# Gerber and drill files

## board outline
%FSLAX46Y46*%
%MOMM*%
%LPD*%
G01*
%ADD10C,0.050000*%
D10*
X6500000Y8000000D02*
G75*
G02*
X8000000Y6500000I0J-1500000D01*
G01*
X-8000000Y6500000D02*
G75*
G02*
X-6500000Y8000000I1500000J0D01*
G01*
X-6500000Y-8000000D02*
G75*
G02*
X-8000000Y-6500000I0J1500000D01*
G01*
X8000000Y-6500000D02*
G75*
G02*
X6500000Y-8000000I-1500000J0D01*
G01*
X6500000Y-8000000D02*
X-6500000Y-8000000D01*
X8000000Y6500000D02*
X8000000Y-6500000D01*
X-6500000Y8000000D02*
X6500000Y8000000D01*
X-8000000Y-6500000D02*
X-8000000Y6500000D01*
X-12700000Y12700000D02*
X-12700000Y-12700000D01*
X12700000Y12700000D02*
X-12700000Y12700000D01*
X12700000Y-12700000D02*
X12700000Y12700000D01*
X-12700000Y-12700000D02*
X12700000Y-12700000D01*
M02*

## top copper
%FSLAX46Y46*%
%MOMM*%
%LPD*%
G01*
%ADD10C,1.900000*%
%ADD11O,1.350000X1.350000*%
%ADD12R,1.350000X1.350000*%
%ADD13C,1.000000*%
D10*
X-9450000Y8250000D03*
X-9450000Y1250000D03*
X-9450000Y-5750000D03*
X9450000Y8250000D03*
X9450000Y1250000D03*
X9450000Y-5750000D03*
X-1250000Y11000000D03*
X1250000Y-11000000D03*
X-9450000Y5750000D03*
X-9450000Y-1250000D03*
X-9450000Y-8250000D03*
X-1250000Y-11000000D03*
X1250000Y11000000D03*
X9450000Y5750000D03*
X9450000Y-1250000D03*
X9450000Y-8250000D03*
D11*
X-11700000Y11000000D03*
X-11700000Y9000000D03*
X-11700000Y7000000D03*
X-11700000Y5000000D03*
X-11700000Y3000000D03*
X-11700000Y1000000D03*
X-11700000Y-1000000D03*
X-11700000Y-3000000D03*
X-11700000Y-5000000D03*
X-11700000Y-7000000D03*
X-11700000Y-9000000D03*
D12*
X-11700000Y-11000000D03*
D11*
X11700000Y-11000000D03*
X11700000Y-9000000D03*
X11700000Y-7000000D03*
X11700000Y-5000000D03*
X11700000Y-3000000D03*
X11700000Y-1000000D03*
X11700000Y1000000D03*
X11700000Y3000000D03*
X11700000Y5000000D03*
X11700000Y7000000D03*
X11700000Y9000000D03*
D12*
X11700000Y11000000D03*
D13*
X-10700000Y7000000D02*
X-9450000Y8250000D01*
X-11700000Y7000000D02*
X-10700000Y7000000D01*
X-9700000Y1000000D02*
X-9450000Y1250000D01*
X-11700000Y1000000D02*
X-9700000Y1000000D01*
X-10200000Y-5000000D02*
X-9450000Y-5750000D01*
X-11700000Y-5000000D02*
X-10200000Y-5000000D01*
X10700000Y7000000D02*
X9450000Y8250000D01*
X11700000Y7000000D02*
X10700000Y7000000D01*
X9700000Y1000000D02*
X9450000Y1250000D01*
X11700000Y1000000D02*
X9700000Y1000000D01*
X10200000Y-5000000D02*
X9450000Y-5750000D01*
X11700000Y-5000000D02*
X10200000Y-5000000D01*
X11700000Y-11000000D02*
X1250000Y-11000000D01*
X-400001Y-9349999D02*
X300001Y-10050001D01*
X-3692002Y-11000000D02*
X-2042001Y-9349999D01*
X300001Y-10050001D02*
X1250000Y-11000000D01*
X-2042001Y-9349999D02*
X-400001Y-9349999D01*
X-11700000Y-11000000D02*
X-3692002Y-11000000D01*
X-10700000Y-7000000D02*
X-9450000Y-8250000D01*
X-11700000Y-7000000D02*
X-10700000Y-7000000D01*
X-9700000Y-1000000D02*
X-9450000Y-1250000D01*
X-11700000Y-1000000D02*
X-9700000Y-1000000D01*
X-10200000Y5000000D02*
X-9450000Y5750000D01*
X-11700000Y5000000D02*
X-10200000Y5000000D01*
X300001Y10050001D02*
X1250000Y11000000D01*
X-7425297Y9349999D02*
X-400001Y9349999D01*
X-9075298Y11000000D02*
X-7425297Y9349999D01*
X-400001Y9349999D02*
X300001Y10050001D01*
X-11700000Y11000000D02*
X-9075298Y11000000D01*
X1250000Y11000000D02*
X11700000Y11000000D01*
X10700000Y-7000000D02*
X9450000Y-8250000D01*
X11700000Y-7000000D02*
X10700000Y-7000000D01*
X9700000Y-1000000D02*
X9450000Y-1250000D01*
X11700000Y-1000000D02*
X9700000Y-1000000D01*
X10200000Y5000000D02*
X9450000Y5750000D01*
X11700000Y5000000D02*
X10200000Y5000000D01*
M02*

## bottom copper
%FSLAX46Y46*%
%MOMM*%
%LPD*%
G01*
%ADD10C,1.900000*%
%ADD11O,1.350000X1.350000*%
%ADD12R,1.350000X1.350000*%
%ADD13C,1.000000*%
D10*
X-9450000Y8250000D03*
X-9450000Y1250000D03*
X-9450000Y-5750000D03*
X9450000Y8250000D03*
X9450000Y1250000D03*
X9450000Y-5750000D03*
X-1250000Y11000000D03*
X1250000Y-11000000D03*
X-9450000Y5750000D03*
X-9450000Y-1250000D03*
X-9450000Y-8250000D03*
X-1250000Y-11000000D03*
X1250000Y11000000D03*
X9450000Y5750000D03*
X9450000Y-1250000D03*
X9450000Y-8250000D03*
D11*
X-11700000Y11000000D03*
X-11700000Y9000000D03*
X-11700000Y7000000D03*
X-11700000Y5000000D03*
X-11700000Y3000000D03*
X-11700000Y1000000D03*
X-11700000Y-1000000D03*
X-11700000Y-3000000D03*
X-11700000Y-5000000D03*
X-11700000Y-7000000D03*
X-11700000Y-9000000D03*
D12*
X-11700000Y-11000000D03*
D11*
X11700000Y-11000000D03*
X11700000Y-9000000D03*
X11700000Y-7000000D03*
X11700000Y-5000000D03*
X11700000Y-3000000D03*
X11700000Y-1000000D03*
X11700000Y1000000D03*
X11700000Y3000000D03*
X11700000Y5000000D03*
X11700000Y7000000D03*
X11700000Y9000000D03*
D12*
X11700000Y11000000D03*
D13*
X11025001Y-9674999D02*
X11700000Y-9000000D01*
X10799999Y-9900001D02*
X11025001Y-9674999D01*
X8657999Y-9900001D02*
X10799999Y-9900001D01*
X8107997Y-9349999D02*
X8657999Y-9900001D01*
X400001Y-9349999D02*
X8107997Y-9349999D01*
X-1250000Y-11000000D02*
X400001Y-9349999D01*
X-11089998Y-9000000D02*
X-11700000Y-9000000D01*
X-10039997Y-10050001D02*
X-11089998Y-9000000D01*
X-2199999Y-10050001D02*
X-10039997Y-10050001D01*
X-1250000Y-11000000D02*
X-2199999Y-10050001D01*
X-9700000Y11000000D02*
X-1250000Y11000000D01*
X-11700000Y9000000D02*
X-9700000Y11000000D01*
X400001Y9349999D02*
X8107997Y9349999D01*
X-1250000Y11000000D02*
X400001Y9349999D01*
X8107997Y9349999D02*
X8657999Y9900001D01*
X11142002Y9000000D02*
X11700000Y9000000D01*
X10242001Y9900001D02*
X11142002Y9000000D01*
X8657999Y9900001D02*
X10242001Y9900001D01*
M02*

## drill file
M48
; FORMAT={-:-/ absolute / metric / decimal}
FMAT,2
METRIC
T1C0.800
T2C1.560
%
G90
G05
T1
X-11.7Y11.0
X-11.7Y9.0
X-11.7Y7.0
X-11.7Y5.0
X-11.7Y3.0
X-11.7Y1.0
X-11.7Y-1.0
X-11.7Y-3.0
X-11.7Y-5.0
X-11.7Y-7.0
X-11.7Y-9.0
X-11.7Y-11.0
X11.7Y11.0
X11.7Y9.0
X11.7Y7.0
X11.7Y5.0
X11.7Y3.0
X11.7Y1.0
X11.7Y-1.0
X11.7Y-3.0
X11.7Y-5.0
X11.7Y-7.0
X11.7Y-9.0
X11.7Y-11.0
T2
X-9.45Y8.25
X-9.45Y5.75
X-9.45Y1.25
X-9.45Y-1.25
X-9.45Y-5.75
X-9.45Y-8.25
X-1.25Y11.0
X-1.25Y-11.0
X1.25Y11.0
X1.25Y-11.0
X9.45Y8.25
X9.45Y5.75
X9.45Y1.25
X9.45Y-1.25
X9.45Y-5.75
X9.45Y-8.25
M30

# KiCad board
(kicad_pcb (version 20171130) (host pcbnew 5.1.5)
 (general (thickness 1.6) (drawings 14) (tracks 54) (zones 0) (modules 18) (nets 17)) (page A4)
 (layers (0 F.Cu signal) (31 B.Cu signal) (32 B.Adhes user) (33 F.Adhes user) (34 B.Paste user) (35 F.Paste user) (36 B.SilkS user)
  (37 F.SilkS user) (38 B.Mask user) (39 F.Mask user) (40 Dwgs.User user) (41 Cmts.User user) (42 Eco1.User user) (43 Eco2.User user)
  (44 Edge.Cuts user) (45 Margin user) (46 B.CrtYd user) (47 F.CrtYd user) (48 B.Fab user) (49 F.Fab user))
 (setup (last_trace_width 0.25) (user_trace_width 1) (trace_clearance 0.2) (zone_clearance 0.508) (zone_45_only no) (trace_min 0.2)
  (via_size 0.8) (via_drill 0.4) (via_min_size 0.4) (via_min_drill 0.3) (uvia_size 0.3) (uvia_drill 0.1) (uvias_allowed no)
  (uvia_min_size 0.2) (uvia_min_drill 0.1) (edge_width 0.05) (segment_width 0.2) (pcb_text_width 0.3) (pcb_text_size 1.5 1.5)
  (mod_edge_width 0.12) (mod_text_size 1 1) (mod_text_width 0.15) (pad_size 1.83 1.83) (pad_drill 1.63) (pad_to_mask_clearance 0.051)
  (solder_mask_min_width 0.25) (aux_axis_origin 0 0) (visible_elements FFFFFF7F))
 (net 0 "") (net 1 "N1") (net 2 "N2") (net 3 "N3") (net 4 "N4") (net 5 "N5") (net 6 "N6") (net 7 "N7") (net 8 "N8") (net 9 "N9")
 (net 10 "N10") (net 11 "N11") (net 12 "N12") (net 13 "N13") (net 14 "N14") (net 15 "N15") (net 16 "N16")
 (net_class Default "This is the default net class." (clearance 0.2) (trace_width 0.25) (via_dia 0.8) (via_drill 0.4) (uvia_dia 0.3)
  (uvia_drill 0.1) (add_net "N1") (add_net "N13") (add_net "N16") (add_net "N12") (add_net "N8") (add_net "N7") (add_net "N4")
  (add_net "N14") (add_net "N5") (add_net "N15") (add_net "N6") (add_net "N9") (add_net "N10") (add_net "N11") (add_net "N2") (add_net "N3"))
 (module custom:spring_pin (layer F.Cu) (at -9.45 -8.25 90)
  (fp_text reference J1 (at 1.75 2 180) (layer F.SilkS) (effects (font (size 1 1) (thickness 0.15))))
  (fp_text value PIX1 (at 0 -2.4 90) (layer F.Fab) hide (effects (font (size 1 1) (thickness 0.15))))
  (pad 1 thru_hole circle (at 0 0 90) (size 1.9 1.9) (drill 1.56) (layers *.Cu *.Mask) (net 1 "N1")))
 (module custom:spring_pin (layer F.Cu) (at -9.45 -1.25 90)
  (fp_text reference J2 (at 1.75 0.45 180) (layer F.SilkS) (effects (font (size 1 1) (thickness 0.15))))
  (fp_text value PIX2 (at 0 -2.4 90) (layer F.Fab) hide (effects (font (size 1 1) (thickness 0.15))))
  (pad 1 thru_hole circle (at 0 0 90) (size 1.9 1.9) (drill 1.56) (layers *.Cu *.Mask) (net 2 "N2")))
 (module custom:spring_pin (layer F.Cu) (at -9.45 5.75 90)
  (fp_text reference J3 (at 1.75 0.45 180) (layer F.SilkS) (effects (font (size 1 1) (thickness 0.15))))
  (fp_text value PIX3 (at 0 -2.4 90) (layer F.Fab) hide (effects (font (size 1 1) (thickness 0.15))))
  (pad 1 thru_hole circle (at 0 0 90) (size 1.9 1.9) (drill 1.56) (layers *.Cu *.Mask) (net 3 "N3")))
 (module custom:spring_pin (layer F.Cu) (at 9.45 -8.25 90)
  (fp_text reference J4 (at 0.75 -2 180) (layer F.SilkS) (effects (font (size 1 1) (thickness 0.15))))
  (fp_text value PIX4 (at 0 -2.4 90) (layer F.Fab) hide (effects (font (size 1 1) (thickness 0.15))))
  (pad 1 thru_hole circle (at 0 0 90) (size 1.9 1.9) (drill 1.56) (layers *.Cu *.Mask) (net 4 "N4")))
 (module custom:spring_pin (layer F.Cu) (at 9.45 -1.25 90)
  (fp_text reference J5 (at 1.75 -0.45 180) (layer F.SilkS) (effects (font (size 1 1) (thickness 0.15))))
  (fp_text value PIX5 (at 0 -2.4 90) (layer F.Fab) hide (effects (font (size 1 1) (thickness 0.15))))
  (pad 1 thru_hole circle (at 0 0 90) (size 1.9 1.9) (drill 1.56) (layers *.Cu *.Mask) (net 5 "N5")))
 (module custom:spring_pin (layer F.Cu) (at 9.45 5.75 90)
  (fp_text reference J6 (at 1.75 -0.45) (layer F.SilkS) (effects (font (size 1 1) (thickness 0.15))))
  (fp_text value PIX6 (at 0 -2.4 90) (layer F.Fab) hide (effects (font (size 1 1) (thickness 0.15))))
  (pad 1 thru_hole circle (at 0 0 90) (size 1.9 1.9) (drill 1.56) (layers *.Cu *.Mask) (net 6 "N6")))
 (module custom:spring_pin (layer F.Cu) (at -1.25 -11 90)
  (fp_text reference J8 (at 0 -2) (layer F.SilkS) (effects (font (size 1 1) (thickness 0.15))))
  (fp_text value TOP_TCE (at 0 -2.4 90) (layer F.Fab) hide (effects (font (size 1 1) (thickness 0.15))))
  (pad 1 thru_hole circle (at 0 0 90) (size 1.9 1.9) (drill 1.56) (layers *.Cu *.Mask) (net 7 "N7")))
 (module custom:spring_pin (layer F.Cu) (at 1.25 11 90)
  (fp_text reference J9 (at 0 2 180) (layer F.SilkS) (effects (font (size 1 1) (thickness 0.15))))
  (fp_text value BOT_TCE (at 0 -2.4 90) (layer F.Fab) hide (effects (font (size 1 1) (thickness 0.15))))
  (pad 1 thru_hole circle (at 0 0 90) (size 1.9 1.9) (drill 1.56) (layers *.Cu *.Mask) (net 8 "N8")))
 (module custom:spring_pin (layer F.Cu) (at -9.45 -5.75 90)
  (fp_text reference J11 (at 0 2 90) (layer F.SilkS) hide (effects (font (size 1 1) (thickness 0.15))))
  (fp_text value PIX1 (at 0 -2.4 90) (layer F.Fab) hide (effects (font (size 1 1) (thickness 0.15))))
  (pad 1 thru_hole circle (at 0 0 90) (size 1.9 1.9) (drill 1.56) (layers *.Cu *.Mask) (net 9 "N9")))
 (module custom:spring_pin (layer F.Cu) (at -9.45 1.25 90)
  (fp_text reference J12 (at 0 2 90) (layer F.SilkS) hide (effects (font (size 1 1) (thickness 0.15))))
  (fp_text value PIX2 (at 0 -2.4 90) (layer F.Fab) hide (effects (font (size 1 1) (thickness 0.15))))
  (pad 1 thru_hole circle (at 0 0 90) (size 1.9 1.9) (drill 1.56) (layers *.Cu *.Mask) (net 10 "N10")))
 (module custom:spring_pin (layer F.Cu) (at -9.45 8.25 90)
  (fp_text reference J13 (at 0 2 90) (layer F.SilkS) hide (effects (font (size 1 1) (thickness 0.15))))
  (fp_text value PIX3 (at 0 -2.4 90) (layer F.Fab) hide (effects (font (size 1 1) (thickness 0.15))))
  (pad 1 thru_hole circle (at 0 0 90) (size 1.9 1.9) (drill 1.56) (layers *.Cu *.Mask) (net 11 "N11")))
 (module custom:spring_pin (layer F.Cu) (at -1.25 11 90)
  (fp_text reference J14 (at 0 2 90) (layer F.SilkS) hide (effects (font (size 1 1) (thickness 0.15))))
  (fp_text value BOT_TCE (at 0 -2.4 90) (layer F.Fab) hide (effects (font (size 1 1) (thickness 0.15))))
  (pad 1 thru_hole circle (at 0 0 90) (size 1.9 1.9) (drill 1.56) (layers *.Cu *.Mask) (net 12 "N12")))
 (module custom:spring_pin (layer F.Cu) (at 1.25 -11 90)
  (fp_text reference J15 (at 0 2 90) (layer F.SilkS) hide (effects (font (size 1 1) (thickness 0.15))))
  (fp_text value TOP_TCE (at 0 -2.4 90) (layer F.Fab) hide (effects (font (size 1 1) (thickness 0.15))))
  (pad 1 thru_hole circle (at 0 0 90) (size 1.9 1.9) (drill 1.56) (layers *.Cu *.Mask) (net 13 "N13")))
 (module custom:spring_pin (layer F.Cu) (at 9.45 -5.75 90)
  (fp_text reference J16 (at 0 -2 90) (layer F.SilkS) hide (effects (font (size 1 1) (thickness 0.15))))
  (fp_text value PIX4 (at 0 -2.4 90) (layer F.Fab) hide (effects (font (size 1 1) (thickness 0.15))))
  (pad 1 thru_hole circle (at 0 0 90) (size 1.9 1.9) (drill 1.56) (layers *.Cu *.Mask) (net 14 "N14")))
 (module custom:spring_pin (layer F.Cu) (at 9.45 1.25 90)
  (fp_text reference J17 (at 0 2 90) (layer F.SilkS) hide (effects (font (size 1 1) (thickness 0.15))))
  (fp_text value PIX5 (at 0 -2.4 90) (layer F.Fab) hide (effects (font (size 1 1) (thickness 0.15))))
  (pad 1 thru_hole circle (at 0 0 90) (size 1.9 1.9) (drill 1.56) (layers *.Cu *.Mask) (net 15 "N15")))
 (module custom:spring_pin (layer F.Cu) (at 9.45 8.25 90)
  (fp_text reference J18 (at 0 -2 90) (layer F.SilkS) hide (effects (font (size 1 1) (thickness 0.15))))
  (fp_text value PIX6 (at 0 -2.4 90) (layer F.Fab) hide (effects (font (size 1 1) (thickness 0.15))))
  (pad 1 thru_hole circle (at 0 0 90) (size 1.9 1.9) (drill 1.56) (layers *.Cu *.Mask) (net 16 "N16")))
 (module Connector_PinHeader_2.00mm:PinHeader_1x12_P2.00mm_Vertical (layer B.Cu) (at -11.7 11)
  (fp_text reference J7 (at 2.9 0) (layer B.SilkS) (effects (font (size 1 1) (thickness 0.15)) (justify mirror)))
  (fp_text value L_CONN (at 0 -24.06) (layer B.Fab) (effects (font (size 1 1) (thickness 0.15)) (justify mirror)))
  (pad 12 thru_hole oval (at 0 -22) (size 1.35 1.35) (drill 0.8) (layers *.Cu *.Mask) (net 13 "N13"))
  (pad 11 thru_hole oval (at 0 -20) (size 1.35 1.35) (drill 0.8) (layers *.Cu *.Mask) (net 7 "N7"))
  (pad 10 thru_hole oval (at 0 -18) (size 1.35 1.35) (drill 0.8) (layers *.Cu *.Mask) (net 1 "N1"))
  (pad 9 thru_hole oval (at 0 -16) (size 1.35 1.35) (drill 0.8) (layers *.Cu *.Mask) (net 9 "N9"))
  (pad 8 thru_hole oval (at 0 -14) (size 1.35 1.35) (drill 0.8) (layers *.Cu *.Mask))
  (pad 7 thru_hole oval (at 0 -12) (size 1.35 1.35) (drill 0.8) (layers *.Cu *.Mask) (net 2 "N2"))
  (pad 6 thru_hole oval (at 0 -10) (size 1.35 1.35) (drill 0.8) (layers *.Cu *.Mask) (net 10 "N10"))
  (pad 5 thru_hole oval (at 0 -8) (size 1.35 1.35) (drill 0.8) (layers *.Cu *.Mask))
  (pad 4 thru_hole oval (at 0 -6) (size 1.35 1.35) (drill 0.8) (layers *.Cu *.Mask) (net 3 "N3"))
  (pad 3 thru_hole oval (at 0 -4) (size 1.35 1.35) (drill 0.8) (layers *.Cu *.Mask) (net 11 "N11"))
  (pad 2 thru_hole oval (at 0 -2) (size 1.35 1.35) (drill 0.8) (layers *.Cu *.Mask) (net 12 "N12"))
  (pad 1 thru_hole rect (at 0 0) (size 1.35 1.35) (drill 0.8) (layers *.Cu *.Mask) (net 8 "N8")))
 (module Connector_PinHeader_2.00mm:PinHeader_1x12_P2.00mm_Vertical (layer B.Cu) (at 11.7 -11 180)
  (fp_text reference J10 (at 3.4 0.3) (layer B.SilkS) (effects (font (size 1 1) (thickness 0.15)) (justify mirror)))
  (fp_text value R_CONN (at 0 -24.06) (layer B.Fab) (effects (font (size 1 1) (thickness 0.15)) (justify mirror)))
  (pad 12 thru_hole oval (at 0 -22 180) (size 1.35 1.35) (drill 0.8) (layers *.Cu *.Mask) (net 8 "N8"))
  (pad 11 thru_hole oval (at 0 -20 180) (size 1.35 1.35) (drill 0.8) (layers *.Cu *.Mask) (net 12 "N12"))
  (pad 10 thru_hole oval (at 0 -18 180) (size 1.35 1.35) (drill 0.8) (layers *.Cu *.Mask) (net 16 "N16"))
  (pad 9 thru_hole oval (at 0 -16 180) (size 1.35 1.35) (drill 0.8) (layers *.Cu *.Mask) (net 6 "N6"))
  (pad 8 thru_hole oval (at 0 -14 180) (size 1.35 1.35) (drill 0.8) (layers *.Cu *.Mask))
  (pad 7 thru_hole oval (at 0 -12 180) (size 1.35 1.35) (drill 0.8) (layers *.Cu *.Mask) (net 15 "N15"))
  (pad 6 thru_hole oval (at 0 -10 180) (size 1.35 1.35) (drill 0.8) (layers *.Cu *.Mask) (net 5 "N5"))
  (pad 5 thru_hole oval (at 0 -8 180) (size 1.35 1.35) (drill 0.8) (layers *.Cu *.Mask))
  (pad 4 thru_hole oval (at 0 -6 180) (size 1.35 1.35) (drill 0.8) (layers *.Cu *.Mask) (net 14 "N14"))
  (pad 3 thru_hole oval (at 0 -4 180) (size 1.35 1.35) (drill 0.8) (layers *.Cu *.Mask) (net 4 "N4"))
  (pad 2 thru_hole oval (at 0 -2 180) (size 1.35 1.35) (drill 0.8) (layers *.Cu *.Mask) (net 7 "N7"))
  (pad 1 thru_hole rect (at 0 0 180) (size 1.35 1.35) (drill 0.8) (layers *.Cu *.Mask) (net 13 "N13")))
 (gr_arc (start 6.5 -6.5) (end 8 -6.5) (angle -90) (layer Edge.Cuts) (width 0.05))
 (gr_arc (start -6.5 -6.5) (end -6.5 -8) (angle -90) (layer Edge.Cuts) (width 0.05))
 (gr_arc (start -6.5 6.5) (end -8 6.5) (angle -90) (layer Edge.Cuts) (width 0.05))
 (gr_arc (start 6.5 6.5) (end 6.5 8) (angle -90) (layer Edge.Cuts) (width 0.05))
 (gr_line (start 6.5 8) (end -6.5 8) (layer Edge.Cuts) (width 0.05))
 (gr_line (start 8 -6.5) (end 8 6.5) (layer Edge.Cuts) (width 0.05))
 (gr_line (start -6.5 -8) (end 6.5 -8) (layer Edge.Cuts) (width 0.05))
 (gr_line (start -8 6.5) (end -8 -6.5) (layer Edge.Cuts) (width 0.05))
 (gr_line (start -12.7 -12.7) (end -12.7 12.7) (layer Edge.Cuts) (width 0.05))
 (gr_line (start 12.7 -12.7) (end -12.7 -12.7) (layer Edge.Cuts) (width 0.05))
 (gr_line (start 12.7 12.7) (end 12.7 -12.7) (layer Edge.Cuts) (width 0.05))
 (gr_line (start -12.7 12.7) (end 12.7 12.7) (layer Edge.Cuts) (width 0.05))
 (segment (start -10.7 -7) (end -9.45 -8.25) (width 1) (layer F.Cu) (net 1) (status 20))
 (segment (start -11.7 -7) (end -10.7 -7) (width 1) (layer F.Cu) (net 1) (status 10))
 (segment (start -9.7 -1) (end -9.45 -1.25) (width 1) (layer F.Cu) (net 2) (status 30))
 (segment (start -11.7 -1) (end -9.7 -1) (width 1) (layer F.Cu) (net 2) (status 30))
 (segment (start -10.2 5) (end -9.45 5.75) (width 1) (layer F.Cu) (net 3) (status 20))
 (segment (start -11.7 5) (end -10.2 5) (width 1) (layer F.Cu) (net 3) (status 10))
 (segment (start 10.7 -7) (end 9.45 -8.25) (width 1) (layer F.Cu) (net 4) (status 20))
 (segment (start 11.7 -7) (end 10.7 -7) (width 1) (layer F.Cu) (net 4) (status 10))
 (segment (start 9.7 -1) (end 9.45 -1.25) (width 1) (layer F.Cu) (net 5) (status 30))
 (segment (start 11.7 -1) (end 9.7 -1) (width 1) (layer F.Cu) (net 5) (status 30))
 (segment (start 10.2 5) (end 9.45 5.75) (width 1) (layer F.Cu) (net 6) (status 20))
 (segment (start 11.7 5) (end 10.2 5) (width 1) (layer F.Cu) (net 6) (status 10))
 (segment (start 11.7 11) (end 1.25 11) (width 1) (layer F.Cu) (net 8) (status 30))
 (segment (start -0.400001 9.349999) (end 0.300001 10.050001) (width 1) (layer F.Cu) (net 8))
 (segment (start -3.692002 11) (end -2.042001 9.349999) (width 1) (layer F.Cu) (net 8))
 (segment (start 0.300001 10.050001) (end 1.25 11) (width 1) (layer F.Cu) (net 8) (status 20))
 (segment (start -2.042001 9.349999) (end -0.400001 9.349999) (width 1) (layer F.Cu) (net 8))
 (segment (start -11.7 11) (end -3.692002 11) (width 1) (layer F.Cu) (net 8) (status 10))
 (segment (start 11.025001 9.674999) (end 11.7 9) (width 1) (layer B.Cu) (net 12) (status 20))
 (segment (start 10.799999 9.900001) (end 11.025001 9.674999) (width 1) (layer B.Cu) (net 12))
 (segment (start 8.657999 9.900001) (end 10.799999 9.900001) (width 1) (layer B.Cu) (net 12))
 (segment (start 8.107997 9.349999) (end 8.657999 9.900001) (width 1) (layer B.Cu) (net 12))
 (segment (start 0.400001 9.349999) (end 8.107997 9.349999) (width 1) (layer B.Cu) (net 12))
 (segment (start -1.25 11) (end 0.400001 9.349999) (width 1) (layer B.Cu) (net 12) (status 10))
 (segment (start -11.089998 9) (end -11.7 9) (width 1) (layer B.Cu) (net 12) (status 30))
 (segment (start -10.039997 10.050001) (end -11.089998 9) (width 1) (layer B.Cu) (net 12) (status 20))
 (segment (start -2.199999 10.050001) (end -10.039997 10.050001) (width 1) (layer B.Cu) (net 12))
 (segment (start -1.25 11) (end -2.199999 10.050001) (width 1) (layer B.Cu) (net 12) (status 10))
 (segment (start -10.7 7) (end -9.45 8.25) (width 1) (layer F.Cu) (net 11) (status 20))
 (segment (start -11.7 7) (end -10.7 7) (width 1) (layer F.Cu) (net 11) (status 10))
 (segment (start -9.7 1) (end -9.45 1.25) (width 1) (layer F.Cu) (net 10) (status 30))
 (segment (start -11.7 1) (end -9.7 1) (width 1) (layer F.Cu) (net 10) (status 30))
 (segment (start -10.2 -5) (end -9.45 -5.75) (width 1) (layer F.Cu) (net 9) (status 20))
 (segment (start -11.7 -5) (end -10.2 -5) (width 1) (layer F.Cu) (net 9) (status 10))
 (segment (start -9.7 -11) (end -1.25 -11) (width 1) (layer B.Cu) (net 7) (status 20))
 (segment (start -11.7 -9) (end -9.7 -11) (width 1) (layer B.Cu) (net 7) (status 10))
 (segment (start 0.400001 -9.349999) (end 8.107997 -9.349999) (width 1) (layer B.Cu) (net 7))
 (segment (start -1.25 -11) (end 0.400001 -9.349999) (width 1) (layer B.Cu) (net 7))
 (segment (start 8.107997 -9.349999) (end 8.657999 -9.900001) (width 1) (layer B.Cu) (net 7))
 (segment (start 11.142002 -9) (end 11.7 -9) (width 1) (layer B.Cu) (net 7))
 (segment (start 10.242001 -9.900001) (end 11.142002 -9) (width 1) (layer B.Cu) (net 7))
 (segment (start 8.657999 -9.900001) (end 10.242001 -9.900001) (width 1) (layer B.Cu) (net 7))
 (segment (start 0.300001 -10.050001) (end 1.25 -11) (width 1) (layer F.Cu) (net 13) (status 20))
 (segment (start -7.425297 -9.349999) (end -0.400001 -9.349999) (width 1) (layer F.Cu) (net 13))
 (segment (start -9.075298 -11) (end -7.425297 -9.349999) (width 1) (layer F.Cu) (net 13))
 (segment (start -0.400001 -9.349999) (end 0.300001 -10.050001) (width 1) (layer F.Cu) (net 13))
 (segment (start -11.7 -11) (end -9.075298 -11) (width 1) (layer F.Cu) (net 13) (status 10))
 (segment (start 1.25 -11) (end 11.7 -11) (width 1) (layer F.Cu) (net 13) (status 30))
 (segment (start 10.7 7) (end 9.45 8.25) (width 1) (layer F.Cu) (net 16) (status 20))
 (segment (start 11.7 7) (end 10.7 7) (width 1) (layer F.Cu) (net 16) (status 10))
 (segment (start 9.7 1) (end 9.45 1.25) (width 1) (layer F.Cu) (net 15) (status 30))
 (segment (start 11.7 1) (end 9.7 1) (width 1) (layer F.Cu) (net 15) (status 30))
 (segment (start 10.2 -5) (end 9.45 -5.75) (width 1) (layer F.Cu) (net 14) (status 20))
 (segment (start 11.7 -5) (end 10.2 -5) (width 1) (layer F.Cu) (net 14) (status 10)))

